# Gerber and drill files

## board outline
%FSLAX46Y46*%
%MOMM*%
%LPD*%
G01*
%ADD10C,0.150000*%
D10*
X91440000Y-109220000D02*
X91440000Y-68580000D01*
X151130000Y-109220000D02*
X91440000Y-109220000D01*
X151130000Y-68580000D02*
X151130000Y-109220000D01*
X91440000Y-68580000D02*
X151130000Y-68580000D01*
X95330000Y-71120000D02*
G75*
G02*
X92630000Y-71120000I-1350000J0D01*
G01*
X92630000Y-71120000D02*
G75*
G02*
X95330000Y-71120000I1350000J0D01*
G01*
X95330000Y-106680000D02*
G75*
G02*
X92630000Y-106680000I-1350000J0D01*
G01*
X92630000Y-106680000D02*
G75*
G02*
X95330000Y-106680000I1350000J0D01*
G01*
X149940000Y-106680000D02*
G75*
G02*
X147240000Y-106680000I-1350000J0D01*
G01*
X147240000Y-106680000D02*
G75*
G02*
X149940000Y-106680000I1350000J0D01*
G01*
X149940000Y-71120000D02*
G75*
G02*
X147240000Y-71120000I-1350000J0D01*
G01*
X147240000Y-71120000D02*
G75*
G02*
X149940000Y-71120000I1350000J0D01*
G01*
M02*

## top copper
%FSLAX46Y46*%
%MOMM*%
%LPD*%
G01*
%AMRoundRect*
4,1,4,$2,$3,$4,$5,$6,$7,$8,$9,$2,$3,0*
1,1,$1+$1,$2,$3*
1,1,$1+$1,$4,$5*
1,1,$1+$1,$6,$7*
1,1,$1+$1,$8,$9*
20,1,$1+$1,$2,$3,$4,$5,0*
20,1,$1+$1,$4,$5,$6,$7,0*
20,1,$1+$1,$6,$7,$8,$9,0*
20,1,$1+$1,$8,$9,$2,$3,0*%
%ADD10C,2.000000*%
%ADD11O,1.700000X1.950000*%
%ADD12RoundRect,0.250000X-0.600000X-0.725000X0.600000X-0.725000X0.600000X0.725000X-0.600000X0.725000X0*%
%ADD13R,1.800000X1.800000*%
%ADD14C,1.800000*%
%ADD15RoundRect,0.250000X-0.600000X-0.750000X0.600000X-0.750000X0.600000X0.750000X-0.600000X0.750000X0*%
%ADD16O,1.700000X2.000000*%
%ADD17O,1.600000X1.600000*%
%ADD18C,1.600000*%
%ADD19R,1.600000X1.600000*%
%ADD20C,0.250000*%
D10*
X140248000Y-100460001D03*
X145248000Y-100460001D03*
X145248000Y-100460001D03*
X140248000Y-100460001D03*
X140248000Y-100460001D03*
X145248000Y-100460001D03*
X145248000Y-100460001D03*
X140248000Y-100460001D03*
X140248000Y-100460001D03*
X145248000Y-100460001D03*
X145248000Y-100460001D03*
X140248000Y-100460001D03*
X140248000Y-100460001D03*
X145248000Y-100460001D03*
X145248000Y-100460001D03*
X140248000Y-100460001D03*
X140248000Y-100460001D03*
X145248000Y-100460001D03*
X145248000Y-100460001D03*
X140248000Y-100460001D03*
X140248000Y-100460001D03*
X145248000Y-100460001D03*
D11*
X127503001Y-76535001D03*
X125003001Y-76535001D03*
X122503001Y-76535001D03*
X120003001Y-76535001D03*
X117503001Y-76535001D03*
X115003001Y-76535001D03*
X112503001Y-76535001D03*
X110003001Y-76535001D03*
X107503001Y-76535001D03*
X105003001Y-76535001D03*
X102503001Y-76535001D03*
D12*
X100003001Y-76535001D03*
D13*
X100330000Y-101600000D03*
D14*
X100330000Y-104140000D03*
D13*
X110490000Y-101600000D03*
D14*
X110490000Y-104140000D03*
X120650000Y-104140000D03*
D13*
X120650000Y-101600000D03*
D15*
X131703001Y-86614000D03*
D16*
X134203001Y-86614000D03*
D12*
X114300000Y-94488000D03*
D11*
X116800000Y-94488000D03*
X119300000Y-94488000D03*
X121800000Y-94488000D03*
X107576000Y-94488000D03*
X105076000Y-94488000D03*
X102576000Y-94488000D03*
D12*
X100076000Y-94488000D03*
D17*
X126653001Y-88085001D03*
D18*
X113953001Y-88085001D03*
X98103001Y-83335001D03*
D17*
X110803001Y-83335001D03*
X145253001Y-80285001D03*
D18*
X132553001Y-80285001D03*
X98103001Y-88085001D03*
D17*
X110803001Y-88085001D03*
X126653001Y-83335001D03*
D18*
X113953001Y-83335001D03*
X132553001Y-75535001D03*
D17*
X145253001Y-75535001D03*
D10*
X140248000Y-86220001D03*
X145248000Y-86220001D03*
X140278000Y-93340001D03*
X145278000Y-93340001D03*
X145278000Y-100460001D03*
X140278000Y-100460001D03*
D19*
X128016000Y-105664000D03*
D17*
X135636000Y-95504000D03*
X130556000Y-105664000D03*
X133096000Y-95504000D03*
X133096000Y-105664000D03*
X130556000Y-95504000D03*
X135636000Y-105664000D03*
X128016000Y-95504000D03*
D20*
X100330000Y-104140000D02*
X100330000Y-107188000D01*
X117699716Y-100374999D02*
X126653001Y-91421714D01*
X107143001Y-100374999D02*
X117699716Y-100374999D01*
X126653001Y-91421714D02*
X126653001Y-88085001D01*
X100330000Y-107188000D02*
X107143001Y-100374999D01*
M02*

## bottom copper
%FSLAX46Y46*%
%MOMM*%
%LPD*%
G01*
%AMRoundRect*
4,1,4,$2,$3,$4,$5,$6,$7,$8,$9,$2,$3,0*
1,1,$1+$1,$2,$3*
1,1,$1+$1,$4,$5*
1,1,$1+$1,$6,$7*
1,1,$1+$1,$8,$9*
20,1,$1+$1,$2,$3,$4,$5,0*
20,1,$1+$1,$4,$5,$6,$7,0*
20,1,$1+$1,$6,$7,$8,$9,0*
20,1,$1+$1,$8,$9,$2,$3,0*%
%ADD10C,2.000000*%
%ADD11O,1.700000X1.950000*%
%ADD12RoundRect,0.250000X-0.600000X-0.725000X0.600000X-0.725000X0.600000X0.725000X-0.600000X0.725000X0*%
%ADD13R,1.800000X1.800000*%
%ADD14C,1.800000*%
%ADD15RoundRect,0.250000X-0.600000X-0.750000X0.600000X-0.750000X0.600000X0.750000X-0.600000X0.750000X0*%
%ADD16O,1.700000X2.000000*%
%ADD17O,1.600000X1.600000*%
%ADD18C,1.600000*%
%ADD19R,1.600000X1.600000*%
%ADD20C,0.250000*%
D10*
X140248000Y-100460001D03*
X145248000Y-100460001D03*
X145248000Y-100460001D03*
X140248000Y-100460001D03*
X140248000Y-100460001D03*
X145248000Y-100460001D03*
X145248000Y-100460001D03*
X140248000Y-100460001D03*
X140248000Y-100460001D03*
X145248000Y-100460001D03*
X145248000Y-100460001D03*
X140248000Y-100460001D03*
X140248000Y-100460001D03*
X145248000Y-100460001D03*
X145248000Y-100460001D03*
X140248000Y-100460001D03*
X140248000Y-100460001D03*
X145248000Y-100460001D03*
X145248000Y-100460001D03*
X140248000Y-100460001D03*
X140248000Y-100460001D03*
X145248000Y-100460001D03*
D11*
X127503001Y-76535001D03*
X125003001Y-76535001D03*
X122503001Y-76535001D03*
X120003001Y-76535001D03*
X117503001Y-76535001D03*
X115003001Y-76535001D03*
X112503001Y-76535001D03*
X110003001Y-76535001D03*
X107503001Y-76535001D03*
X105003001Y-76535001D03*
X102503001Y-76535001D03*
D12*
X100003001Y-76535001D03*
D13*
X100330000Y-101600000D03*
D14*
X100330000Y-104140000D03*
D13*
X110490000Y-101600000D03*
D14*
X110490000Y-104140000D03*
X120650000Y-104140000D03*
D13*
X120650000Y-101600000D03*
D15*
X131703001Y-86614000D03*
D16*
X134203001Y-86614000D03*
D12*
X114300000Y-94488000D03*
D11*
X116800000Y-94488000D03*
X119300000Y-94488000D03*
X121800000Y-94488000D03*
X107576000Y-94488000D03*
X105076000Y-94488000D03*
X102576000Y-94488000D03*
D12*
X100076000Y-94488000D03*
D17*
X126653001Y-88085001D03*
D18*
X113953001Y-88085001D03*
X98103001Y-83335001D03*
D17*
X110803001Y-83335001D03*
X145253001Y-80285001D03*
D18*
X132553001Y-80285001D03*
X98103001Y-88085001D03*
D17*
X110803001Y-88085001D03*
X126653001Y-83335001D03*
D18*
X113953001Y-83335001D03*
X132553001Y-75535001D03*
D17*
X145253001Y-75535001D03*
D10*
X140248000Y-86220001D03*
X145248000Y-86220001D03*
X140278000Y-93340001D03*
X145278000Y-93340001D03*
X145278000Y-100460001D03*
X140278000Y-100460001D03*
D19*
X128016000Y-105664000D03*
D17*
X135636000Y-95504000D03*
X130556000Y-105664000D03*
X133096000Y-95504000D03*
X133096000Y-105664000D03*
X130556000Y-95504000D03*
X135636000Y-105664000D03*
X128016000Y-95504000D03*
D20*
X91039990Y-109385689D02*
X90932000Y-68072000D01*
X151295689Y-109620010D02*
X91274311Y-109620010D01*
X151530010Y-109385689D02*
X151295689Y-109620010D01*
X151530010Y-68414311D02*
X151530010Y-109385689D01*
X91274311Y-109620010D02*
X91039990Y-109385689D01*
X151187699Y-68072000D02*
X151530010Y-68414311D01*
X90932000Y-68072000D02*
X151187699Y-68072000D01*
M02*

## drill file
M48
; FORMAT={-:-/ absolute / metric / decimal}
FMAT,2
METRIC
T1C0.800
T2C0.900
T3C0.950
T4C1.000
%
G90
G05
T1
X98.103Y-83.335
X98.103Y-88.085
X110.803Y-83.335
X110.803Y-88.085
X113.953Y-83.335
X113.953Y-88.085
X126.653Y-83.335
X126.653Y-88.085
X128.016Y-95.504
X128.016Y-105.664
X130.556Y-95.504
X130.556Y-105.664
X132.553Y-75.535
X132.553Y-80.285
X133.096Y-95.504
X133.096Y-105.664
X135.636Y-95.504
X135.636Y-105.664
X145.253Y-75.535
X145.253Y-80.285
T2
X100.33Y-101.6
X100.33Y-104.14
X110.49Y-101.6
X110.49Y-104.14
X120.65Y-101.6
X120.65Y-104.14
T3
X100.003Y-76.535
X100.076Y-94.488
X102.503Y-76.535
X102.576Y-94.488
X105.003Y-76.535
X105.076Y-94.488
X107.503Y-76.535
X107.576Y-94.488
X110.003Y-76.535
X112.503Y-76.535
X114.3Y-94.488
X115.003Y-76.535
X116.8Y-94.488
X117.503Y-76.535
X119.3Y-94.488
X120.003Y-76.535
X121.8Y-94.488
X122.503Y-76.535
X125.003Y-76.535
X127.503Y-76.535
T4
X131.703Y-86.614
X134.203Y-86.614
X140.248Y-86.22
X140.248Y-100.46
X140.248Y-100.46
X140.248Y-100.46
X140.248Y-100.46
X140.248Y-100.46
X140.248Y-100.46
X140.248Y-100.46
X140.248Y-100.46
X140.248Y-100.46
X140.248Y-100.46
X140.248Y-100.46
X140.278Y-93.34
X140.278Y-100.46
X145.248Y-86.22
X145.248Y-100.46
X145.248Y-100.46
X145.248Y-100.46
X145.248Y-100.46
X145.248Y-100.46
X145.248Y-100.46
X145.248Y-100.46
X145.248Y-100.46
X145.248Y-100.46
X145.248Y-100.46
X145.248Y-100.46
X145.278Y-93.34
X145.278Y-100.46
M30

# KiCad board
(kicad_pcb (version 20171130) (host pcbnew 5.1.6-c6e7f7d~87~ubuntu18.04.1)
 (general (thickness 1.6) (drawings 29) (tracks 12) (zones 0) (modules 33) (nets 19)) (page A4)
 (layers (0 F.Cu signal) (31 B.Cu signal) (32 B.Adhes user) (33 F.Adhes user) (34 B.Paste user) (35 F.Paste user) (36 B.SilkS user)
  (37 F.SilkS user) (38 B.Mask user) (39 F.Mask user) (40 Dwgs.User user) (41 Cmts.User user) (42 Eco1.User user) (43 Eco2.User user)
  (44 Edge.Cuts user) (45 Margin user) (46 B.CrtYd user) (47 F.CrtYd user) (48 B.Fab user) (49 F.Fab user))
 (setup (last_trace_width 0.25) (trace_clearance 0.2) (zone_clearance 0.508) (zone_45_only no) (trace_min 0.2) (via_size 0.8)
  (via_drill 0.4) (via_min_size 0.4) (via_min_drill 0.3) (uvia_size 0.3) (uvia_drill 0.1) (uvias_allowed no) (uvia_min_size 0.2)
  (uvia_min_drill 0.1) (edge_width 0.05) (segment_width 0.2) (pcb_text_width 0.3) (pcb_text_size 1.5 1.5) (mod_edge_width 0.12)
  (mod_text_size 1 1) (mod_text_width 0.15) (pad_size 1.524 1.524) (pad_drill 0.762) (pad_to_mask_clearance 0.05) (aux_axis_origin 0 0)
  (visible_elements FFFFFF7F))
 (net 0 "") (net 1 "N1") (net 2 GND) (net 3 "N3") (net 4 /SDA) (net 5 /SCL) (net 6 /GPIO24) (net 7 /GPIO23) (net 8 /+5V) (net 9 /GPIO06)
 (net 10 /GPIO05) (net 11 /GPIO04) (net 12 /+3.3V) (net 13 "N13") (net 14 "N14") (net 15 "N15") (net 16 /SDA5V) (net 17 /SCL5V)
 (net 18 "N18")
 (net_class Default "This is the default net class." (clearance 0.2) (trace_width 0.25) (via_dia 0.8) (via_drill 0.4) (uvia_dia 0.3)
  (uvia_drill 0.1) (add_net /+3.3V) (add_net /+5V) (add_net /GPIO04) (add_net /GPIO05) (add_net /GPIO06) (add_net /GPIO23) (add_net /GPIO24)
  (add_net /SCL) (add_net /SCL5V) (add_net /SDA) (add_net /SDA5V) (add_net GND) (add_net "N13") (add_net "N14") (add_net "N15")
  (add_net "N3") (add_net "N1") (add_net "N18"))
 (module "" (layer F.Cu) (at 128.524 85.852)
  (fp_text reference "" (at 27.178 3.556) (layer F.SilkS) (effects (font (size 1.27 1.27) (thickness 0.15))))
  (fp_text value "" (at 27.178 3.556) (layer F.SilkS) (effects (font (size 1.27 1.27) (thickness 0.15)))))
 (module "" (layer F.Cu) (at 27.178 3.556)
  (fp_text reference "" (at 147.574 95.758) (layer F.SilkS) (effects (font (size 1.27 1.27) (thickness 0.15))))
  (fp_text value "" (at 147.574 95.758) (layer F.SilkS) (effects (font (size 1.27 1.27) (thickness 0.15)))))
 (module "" (layer F.Cu) (at 147.32 88.392)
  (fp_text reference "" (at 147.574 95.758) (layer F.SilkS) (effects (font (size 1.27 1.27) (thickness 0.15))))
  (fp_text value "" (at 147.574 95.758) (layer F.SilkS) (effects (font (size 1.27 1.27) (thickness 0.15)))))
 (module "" (layer F.Cu) (at 147.574 95.758)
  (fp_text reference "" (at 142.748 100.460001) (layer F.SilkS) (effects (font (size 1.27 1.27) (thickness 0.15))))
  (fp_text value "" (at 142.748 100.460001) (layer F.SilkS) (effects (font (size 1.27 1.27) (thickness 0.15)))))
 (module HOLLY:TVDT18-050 (layer F.Cu) (at 142.748 100.460001)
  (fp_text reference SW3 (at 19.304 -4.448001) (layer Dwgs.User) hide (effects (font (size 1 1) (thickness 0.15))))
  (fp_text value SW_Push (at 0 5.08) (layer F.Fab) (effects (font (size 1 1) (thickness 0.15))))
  (pad 1 thru_hole circle (at -2.5 0) (size 2 2) (drill 1) (layers *.Cu *.Mask) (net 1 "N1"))
  (pad 2 thru_hole circle (at 2.5 0) (size 2 2) (drill 1) (layers *.Cu *.Mask) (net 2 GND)))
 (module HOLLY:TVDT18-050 (layer F.Cu) (at 142.748 100.460001)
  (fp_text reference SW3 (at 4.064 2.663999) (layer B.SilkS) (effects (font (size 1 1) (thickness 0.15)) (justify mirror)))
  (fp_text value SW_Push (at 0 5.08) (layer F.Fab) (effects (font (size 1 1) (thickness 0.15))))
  (pad 2 thru_hole circle (at 2.5 0) (size 2 2) (drill 1) (layers *.Cu *.Mask) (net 2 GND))
  (pad 1 thru_hole circle (at -2.5 0) (size 2 2) (drill 1) (layers *.Cu *.Mask) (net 1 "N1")))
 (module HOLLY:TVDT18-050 (layer F.Cu) (at 142.748 100.460001)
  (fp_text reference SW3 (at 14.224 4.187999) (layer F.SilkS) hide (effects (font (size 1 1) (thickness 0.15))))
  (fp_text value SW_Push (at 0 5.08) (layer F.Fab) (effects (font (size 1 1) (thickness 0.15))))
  (pad 1 thru_hole circle (at -2.5 0) (size 2 2) (drill 1) (layers *.Cu *.Mask) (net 1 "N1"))
  (pad 2 thru_hole circle (at 2.5 0) (size 2 2) (drill 1) (layers *.Cu *.Mask) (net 2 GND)))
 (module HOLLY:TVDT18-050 (layer F.Cu) (at 142.748 100.460001)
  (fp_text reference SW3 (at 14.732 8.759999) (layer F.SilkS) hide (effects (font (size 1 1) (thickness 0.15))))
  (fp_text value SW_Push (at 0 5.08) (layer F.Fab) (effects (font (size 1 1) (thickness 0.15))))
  (pad 2 thru_hole circle (at 2.5 0) (size 2 2) (drill 1) (layers *.Cu *.Mask) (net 2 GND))
  (pad 1 thru_hole circle (at -2.5 0) (size 2 2) (drill 1) (layers *.Cu *.Mask) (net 1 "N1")))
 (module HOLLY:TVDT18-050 (layer F.Cu) (at 142.748 100.460001)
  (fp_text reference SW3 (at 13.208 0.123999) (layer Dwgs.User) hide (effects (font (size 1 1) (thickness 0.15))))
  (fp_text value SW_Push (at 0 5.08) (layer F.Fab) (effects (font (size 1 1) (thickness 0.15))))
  (pad 1 thru_hole circle (at -2.5 0) (size 2 2) (drill 1) (layers *.Cu *.Mask) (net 1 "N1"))
  (pad 2 thru_hole circle (at 2.5 0) (size 2 2) (drill 1) (layers *.Cu *.Mask) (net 2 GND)))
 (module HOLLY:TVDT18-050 (layer F.Cu) (at 142.748 100.460001)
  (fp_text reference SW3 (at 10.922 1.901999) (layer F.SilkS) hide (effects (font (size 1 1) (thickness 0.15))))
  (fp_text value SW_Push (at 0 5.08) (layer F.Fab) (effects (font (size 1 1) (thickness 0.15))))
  (pad 2 thru_hole circle (at 2.5 0) (size 2 2) (drill 1) (layers *.Cu *.Mask) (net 2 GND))
  (pad 1 thru_hole circle (at -2.5 0) (size 2 2) (drill 1) (layers *.Cu *.Mask) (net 1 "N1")))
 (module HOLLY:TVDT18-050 (layer F.Cu) (at 142.748 100.460001)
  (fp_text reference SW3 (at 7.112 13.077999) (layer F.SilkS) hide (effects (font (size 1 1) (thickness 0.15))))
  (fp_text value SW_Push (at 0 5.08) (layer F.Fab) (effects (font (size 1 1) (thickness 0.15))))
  (pad 1 thru_hole circle (at -2.5 0) (size 2 2) (drill 1) (layers *.Cu *.Mask) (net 1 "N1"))
  (pad 2 thru_hole circle (at 2.5 0) (size 2 2) (drill 1) (layers *.Cu *.Mask) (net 2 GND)))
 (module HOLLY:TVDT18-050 (layer F.Cu) (at 142.748 100.460001)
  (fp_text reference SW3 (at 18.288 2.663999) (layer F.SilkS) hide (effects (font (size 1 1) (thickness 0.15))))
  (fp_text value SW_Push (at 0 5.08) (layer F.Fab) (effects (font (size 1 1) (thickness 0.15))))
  (pad 2 thru_hole circle (at 2.5 0) (size 2 2) (drill 1) (layers *.Cu *.Mask) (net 2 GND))
  (pad 1 thru_hole circle (at -2.5 0) (size 2 2) (drill 1) (layers *.Cu *.Mask) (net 1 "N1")))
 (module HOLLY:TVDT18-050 (layer F.Cu) (at 142.748 100.460001)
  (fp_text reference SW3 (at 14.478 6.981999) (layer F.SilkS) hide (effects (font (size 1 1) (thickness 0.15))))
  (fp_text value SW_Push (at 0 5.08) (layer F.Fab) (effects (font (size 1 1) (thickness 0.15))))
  (pad 1 thru_hole circle (at -2.5 0) (size 2 2) (drill 1) (layers *.Cu *.Mask) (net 1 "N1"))
  (pad 2 thru_hole circle (at 2.5 0) (size 2 2) (drill 1) (layers *.Cu *.Mask) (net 2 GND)))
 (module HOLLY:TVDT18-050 (layer F.Cu) (at 142.748 100.460001)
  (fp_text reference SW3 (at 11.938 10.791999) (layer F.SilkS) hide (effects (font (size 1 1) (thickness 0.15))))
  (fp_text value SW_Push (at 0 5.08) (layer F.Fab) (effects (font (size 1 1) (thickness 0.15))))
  (pad 2 thru_hole circle (at 2.5 0) (size 2 2) (drill 1) (layers *.Cu *.Mask) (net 2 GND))
  (pad 1 thru_hole circle (at -2.5 0) (size 2 2) (drill 1) (layers *.Cu *.Mask) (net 1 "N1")))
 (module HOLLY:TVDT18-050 (layer F.Cu) (at 142.748 100.460001)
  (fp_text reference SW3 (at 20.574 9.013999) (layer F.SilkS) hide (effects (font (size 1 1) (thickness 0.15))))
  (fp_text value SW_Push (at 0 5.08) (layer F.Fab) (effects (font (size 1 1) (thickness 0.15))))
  (pad 1 thru_hole circle (at -2.5 0) (size 2 2) (drill 1) (layers *.Cu *.Mask) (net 1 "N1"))
  (pad 2 thru_hole circle (at 2.5 0) (size 2 2) (drill 1) (layers *.Cu *.Mask) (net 2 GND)))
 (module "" (layer F.Cu) (at 103.632 102.108)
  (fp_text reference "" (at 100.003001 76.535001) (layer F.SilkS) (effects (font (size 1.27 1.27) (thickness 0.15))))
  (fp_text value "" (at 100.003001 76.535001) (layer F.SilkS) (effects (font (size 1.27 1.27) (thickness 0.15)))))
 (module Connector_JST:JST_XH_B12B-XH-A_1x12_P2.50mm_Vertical (layer F.Cu) (at 100.003001 76.535001)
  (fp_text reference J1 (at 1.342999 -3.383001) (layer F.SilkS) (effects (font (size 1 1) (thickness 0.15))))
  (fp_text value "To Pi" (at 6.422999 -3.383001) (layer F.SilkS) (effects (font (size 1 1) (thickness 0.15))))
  (pad 12 thru_hole oval (at 27.5 0) (size 1.7 1.95) (drill 0.95) (layers *.Cu *.Mask) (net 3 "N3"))
  (pad 11 thru_hole oval (at 25 0) (size 1.7 1.95) (drill 0.95) (layers *.Cu *.Mask) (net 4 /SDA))
  (pad 10 thru_hole oval (at 22.5 0) (size 1.7 1.95) (drill 0.95) (layers *.Cu *.Mask) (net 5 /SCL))
  (pad 9 thru_hole oval (at 20 0) (size 1.7 1.95) (drill 0.95) (layers *.Cu *.Mask) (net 1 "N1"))
  (pad 8 thru_hole oval (at 17.5 0) (size 1.7 1.95) (drill 0.95) (layers *.Cu *.Mask) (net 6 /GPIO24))
  (pad 7 thru_hole oval (at 15 0) (size 1.7 1.95) (drill 0.95) (layers *.Cu *.Mask) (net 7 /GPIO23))
  (pad 6 thru_hole oval (at 12.5 0) (size 1.7 1.95) (drill 0.95) (layers *.Cu *.Mask) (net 2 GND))
  (pad 5 thru_hole oval (at 10 0) (size 1.7 1.95) (drill 0.95) (layers *.Cu *.Mask) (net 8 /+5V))
  (pad 4 thru_hole oval (at 7.5 0) (size 1.7 1.95) (drill 0.95) (layers *.Cu *.Mask) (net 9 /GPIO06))
  (pad 3 thru_hole oval (at 5 0) (size 1.7 1.95) (drill 0.95) (layers *.Cu *.Mask) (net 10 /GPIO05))
  (pad 2 thru_hole oval (at 2.5 0) (size 1.7 1.95) (drill 0.95) (layers *.Cu *.Mask) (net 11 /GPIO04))
  (pad 1 thru_hole roundrect (at 0 0) (size 1.7 1.95) (drill 0.95) (layers *.Cu *.Mask) (roundrect_rratio 0.147059) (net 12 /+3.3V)))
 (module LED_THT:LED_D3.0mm (layer B.Cu) (at 100.33 101.6 270)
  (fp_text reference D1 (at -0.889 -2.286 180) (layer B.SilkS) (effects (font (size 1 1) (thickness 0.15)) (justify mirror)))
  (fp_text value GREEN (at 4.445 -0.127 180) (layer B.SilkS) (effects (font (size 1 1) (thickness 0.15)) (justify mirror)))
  (pad 1 thru_hole rect (at 0 0 270) (size 1.8 1.8) (drill 0.9) (layers *.Cu *.Mask) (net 11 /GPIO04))
  (pad 2 thru_hole circle (at 2.54 0 270) (size 1.8 1.8) (drill 0.9) (layers *.Cu *.Mask) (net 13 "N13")))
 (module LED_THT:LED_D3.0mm (layer B.Cu) (at 110.49 101.6 270)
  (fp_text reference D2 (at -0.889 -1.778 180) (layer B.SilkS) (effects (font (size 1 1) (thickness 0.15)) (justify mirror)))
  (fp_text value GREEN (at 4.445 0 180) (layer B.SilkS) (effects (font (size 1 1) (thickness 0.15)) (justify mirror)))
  (pad 1 thru_hole rect (at 0 0 270) (size 1.8 1.8) (drill 0.9) (layers *.Cu *.Mask) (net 10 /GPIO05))
  (pad 2 thru_hole circle (at 2.54 0 270) (size 1.8 1.8) (drill 0.9) (layers *.Cu *.Mask) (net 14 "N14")))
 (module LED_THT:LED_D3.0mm (layer B.Cu) (at 120.65 101.6 270)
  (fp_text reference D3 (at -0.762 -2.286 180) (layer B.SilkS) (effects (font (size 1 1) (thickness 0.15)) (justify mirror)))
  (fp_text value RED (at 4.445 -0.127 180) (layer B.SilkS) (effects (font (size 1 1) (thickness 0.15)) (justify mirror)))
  (pad 2 thru_hole circle (at 2.54 0 270) (size 1.8 1.8) (drill 0.9) (layers *.Cu *.Mask) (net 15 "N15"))
  (pad 1 thru_hole rect (at 0 0 270) (size 1.8 1.8) (drill 0.9) (layers *.Cu *.Mask) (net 9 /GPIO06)))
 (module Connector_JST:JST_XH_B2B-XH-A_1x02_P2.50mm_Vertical (layer F.Cu) (at 131.703001 86.614)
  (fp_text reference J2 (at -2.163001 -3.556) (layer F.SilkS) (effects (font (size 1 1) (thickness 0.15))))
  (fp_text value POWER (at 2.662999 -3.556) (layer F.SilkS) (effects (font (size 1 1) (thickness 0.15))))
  (pad 1 thru_hole roundrect (at 0 0) (size 1.7 2) (drill 1) (layers *.Cu *.Mask) (roundrect_rratio 0.147059) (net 8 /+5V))
  (pad 2 thru_hole oval (at 2.5 0) (size 1.7 2) (drill 1) (layers *.Cu *.Mask) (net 2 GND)))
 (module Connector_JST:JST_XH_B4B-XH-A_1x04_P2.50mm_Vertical (layer F.Cu) (at 114.3 94.488)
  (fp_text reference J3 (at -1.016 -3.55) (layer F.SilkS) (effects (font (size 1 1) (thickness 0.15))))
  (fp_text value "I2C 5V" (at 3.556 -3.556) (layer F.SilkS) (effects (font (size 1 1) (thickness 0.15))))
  (pad 1 thru_hole roundrect (at 0 0) (size 1.7 1.95) (drill 0.95) (layers *.Cu *.Mask) (roundrect_rratio 0.147059) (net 2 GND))
  (pad 2 thru_hole oval (at 2.5 0) (size 1.7 1.95) (drill 0.95) (layers *.Cu *.Mask) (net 8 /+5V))
  (pad 3 thru_hole oval (at 5 0) (size 1.7 1.95) (drill 0.95) (layers *.Cu *.Mask) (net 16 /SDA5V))
  (pad 4 thru_hole oval (at 7.5 0) (size 1.7 1.95) (drill 0.95) (layers *.Cu *.Mask) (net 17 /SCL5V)))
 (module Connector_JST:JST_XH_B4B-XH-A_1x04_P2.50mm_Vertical (layer F.Cu) (at 100.076 94.488)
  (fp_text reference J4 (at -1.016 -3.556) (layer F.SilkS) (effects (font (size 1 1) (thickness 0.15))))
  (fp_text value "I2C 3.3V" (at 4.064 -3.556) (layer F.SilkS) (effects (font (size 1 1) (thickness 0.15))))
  (pad 4 thru_hole oval (at 7.5 0) (size 1.7 1.95) (drill 0.95) (layers *.Cu *.Mask) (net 5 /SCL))
  (pad 3 thru_hole oval (at 5 0) (size 1.7 1.95) (drill 0.95) (layers *.Cu *.Mask) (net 4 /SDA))
  (pad 2 thru_hole oval (at 2.5 0) (size 1.7 1.95) (drill 0.95) (layers *.Cu *.Mask) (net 12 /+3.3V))
  (pad 1 thru_hole roundrect (at 0 0) (size 1.7 1.95) (drill 0.95) (layers *.Cu *.Mask) (roundrect_rratio 0.147059) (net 2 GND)))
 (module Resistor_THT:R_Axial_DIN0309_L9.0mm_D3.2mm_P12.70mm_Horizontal (layer F.Cu) (at 113.953001 88.085001)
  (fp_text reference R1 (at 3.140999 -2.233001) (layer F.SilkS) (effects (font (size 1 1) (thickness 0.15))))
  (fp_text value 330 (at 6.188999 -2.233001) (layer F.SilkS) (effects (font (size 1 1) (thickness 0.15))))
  (pad 2 thru_hole oval (at 12.7 0) (size 1.6 1.6) (drill 0.8) (layers *.Cu *.Mask) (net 13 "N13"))
  (pad 1 thru_hole circle (at 0 0) (size 1.6 1.6) (drill 0.8) (layers *.Cu *.Mask) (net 12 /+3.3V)))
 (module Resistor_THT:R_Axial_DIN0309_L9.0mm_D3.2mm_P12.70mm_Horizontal (layer F.Cu) (at 98.103001 83.335001)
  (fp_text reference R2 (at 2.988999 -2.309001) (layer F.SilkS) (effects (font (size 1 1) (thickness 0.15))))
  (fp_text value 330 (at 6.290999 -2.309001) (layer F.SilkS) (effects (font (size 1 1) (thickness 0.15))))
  (pad 1 thru_hole circle (at 0 0) (size 1.6 1.6) (drill 0.8) (layers *.Cu *.Mask) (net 12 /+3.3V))
  (pad 2 thru_hole oval (at 12.7 0) (size 1.6 1.6) (drill 0.8) (layers *.Cu *.Mask) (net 14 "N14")))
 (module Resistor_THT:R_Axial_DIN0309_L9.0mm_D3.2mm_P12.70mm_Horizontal (layer F.Cu) (at 132.553001 80.285001)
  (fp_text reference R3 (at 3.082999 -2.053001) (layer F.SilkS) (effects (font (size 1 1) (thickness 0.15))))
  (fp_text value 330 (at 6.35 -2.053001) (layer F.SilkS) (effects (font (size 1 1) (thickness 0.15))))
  (pad 2 thru_hole oval (at 12.7 0) (size 1.6 1.6) (drill 0.8) (layers *.Cu *.Mask) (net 15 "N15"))
  (pad 1 thru_hole circle (at 0 0) (size 1.6 1.6) (drill 0.8) (layers *.Cu *.Mask) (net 12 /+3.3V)))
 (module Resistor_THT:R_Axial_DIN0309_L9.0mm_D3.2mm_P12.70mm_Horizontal (layer F.Cu) (at 98.103001 88.085001)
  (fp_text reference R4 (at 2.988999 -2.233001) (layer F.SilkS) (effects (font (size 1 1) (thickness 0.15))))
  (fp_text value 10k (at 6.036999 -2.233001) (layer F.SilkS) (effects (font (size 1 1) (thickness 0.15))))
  (pad 1 thru_hole circle (at 0 0) (size 1.6 1.6) (drill 0.8) (layers *.Cu *.Mask) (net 12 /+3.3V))
  (pad 2 thru_hole oval (at 12.7 0) (size 1.6 1.6) (drill 0.8) (layers *.Cu *.Mask) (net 7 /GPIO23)))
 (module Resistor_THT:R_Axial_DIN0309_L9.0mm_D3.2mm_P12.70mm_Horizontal (layer F.Cu) (at 113.953001 83.335001)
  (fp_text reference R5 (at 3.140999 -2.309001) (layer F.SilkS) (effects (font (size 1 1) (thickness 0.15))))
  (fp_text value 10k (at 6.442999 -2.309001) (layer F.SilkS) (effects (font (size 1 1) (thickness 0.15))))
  (pad 2 thru_hole oval (at 12.7 0) (size 1.6 1.6) (drill 0.8) (layers *.Cu *.Mask) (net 6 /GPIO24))
  (pad 1 thru_hole circle (at 0 0) (size 1.6 1.6) (drill 0.8) (layers *.Cu *.Mask) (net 12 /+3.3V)))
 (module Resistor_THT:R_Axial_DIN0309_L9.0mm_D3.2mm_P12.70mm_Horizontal (layer F.Cu) (at 132.553001 75.535001)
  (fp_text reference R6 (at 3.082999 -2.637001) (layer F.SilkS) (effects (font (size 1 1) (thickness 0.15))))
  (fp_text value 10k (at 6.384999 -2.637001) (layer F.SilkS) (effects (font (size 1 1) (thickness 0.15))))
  (pad 1 thru_hole circle (at 0 0) (size 1.6 1.6) (drill 0.8) (layers *.Cu *.Mask) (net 12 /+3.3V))
  (pad 2 thru_hole oval (at 12.7 0) (size 1.6 1.6) (drill 0.8) (layers *.Cu *.Mask) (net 1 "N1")))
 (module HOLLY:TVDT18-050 (layer F.Cu) (at 142.748 86.220001)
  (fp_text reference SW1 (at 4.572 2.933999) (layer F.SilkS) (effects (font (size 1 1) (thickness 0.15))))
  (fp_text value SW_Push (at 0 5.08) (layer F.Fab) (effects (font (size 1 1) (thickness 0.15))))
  (pad 1 thru_hole circle (at -2.5 0) (size 2 2) (drill 1) (layers *.Cu *.Mask) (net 7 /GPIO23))
  (pad 2 thru_hole circle (at 2.5 0) (size 2 2) (drill 1) (layers *.Cu *.Mask) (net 2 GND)))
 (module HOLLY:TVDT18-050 (layer F.Cu) (at 142.778 93.340001)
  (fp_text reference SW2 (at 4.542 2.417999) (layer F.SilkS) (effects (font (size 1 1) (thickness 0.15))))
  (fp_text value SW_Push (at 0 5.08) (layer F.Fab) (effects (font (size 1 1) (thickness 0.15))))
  (pad 1 thru_hole circle (at -2.5 0) (size 2 2) (drill 1) (layers *.Cu *.Mask) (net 6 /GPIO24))
  (pad 2 thru_hole circle (at 2.5 0) (size 2 2) (drill 1) (layers *.Cu *.Mask) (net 2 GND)))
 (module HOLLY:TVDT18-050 (layer F.Cu) (at 142.778 100.460001)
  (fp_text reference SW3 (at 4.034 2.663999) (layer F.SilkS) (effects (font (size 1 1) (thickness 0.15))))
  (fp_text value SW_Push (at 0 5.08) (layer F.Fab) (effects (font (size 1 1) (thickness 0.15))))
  (pad 2 thru_hole circle (at 2.5 0) (size 2 2) (drill 1) (layers *.Cu *.Mask) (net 2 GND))
  (pad 1 thru_hole circle (at -2.5 0) (size 2 2) (drill 1) (layers *.Cu *.Mask) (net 1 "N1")))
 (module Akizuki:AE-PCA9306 (layer F.Cu) (at 128.016 105.664 90)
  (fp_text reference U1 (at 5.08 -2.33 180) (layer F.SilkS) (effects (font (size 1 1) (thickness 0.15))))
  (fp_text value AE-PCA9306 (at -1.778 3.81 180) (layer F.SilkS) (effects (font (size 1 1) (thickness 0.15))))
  (pad 1 thru_hole rect (at 0 0 90) (size 1.6 1.6) (drill 0.8) (layers *.Cu *.Mask) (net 12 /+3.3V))
  (pad 5 thru_hole oval (at 10.16 7.62 90) (size 1.6 1.6) (drill 0.8) (layers *.Cu *.Mask) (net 2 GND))
  (pad 2 thru_hole oval (at 0 2.54 90) (size 1.6 1.6) (drill 0.8) (layers *.Cu *.Mask) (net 5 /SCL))
  (pad 6 thru_hole oval (at 10.16 5.08 90) (size 1.6 1.6) (drill 0.8) (layers *.Cu *.Mask) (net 16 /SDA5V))
  (pad 3 thru_hole oval (at 0 5.08 90) (size 1.6 1.6) (drill 0.8) (layers *.Cu *.Mask) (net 4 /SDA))
  (pad 7 thru_hole oval (at 10.16 2.54 90) (size 1.6 1.6) (drill 0.8) (layers *.Cu *.Mask) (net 17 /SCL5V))
  (pad 4 thru_hole oval (at 0 7.62 90) (size 1.6 1.6) (drill 0.8) (layers *.Cu *.Mask) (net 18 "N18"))
  (pad 8 thru_hole oval (at 10.16 0 90) (size 1.6 1.6) (drill 0.8) (layers *.Cu *.Mask) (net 8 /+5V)))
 (gr_line (start 91.44 109.22) (end 91.44 68.58) (layer Edge.Cuts) (width 0.15))
 (gr_line (start 151.13 109.22) (end 91.44 109.22) (layer Edge.Cuts) (width 0.15))
 (gr_line (start 151.13 68.58) (end 151.13 109.22) (layer Edge.Cuts) (width 0.15))
 (gr_line (start 91.44 68.58) (end 151.13 68.58) (layer Edge.Cuts) (width 0.15))
 (gr_circle (center 93.98 71.12) (end 95.33 71.12) (layer Edge.Cuts) (width 0.15))
 (gr_circle (center 93.98 106.68) (end 95.33 106.68) (layer Edge.Cuts) (width 0.15))
 (gr_circle (center 148.59 106.68) (end 149.94 106.68) (layer Edge.Cuts) (width 0.15))
 (gr_circle (center 148.59 71.12) (end 149.94 71.12) (layer Edge.Cuts) (width 0.15))
 (segment (start 91.03999 109.385689) (end 90.932 68.072) (width 0.25) (layer B.Cu) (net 2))
 (segment (start 151.295689 109.62001) (end 91.274311 109.62001) (width 0.25) (layer B.Cu) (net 2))
 (segment (start 151.53001 109.385689) (end 151.295689 109.62001) (width 0.25) (layer B.Cu) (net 2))
 (segment (start 151.53001 68.414311) (end 151.53001 109.385689) (width 0.25) (layer B.Cu) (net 2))
 (segment (start 91.274311 109.62001) (end 91.03999 109.385689) (width 0.25) (layer B.Cu) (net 2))
 (segment (start 151.187699 68.072) (end 151.53001 68.414311) (width 0.25) (layer B.Cu) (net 2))
 (segment (start 90.932 68.072) (end 151.187699 68.072) (width 0.25) (layer B.Cu) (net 2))
 (segment (start 100.33 104.14) (end 100.33 107.188) (width 0.25) (layer F.Cu) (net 13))
 (segment (start 117.699716 100.374999) (end 126.653001 91.421714) (width 0.25) (layer F.Cu) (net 13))
 (segment (start 107.143001 100.374999) (end 117.699716 100.374999) (width 0.25) (layer F.Cu) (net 13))
 (segment (start 126.653001 91.421714) (end 126.653001 88.085001) (width 0.25) (layer F.Cu) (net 13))
 (segment (start 100.33 107.188) (end 107.143001 100.374999) (width 0.25) (layer F.Cu) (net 13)))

